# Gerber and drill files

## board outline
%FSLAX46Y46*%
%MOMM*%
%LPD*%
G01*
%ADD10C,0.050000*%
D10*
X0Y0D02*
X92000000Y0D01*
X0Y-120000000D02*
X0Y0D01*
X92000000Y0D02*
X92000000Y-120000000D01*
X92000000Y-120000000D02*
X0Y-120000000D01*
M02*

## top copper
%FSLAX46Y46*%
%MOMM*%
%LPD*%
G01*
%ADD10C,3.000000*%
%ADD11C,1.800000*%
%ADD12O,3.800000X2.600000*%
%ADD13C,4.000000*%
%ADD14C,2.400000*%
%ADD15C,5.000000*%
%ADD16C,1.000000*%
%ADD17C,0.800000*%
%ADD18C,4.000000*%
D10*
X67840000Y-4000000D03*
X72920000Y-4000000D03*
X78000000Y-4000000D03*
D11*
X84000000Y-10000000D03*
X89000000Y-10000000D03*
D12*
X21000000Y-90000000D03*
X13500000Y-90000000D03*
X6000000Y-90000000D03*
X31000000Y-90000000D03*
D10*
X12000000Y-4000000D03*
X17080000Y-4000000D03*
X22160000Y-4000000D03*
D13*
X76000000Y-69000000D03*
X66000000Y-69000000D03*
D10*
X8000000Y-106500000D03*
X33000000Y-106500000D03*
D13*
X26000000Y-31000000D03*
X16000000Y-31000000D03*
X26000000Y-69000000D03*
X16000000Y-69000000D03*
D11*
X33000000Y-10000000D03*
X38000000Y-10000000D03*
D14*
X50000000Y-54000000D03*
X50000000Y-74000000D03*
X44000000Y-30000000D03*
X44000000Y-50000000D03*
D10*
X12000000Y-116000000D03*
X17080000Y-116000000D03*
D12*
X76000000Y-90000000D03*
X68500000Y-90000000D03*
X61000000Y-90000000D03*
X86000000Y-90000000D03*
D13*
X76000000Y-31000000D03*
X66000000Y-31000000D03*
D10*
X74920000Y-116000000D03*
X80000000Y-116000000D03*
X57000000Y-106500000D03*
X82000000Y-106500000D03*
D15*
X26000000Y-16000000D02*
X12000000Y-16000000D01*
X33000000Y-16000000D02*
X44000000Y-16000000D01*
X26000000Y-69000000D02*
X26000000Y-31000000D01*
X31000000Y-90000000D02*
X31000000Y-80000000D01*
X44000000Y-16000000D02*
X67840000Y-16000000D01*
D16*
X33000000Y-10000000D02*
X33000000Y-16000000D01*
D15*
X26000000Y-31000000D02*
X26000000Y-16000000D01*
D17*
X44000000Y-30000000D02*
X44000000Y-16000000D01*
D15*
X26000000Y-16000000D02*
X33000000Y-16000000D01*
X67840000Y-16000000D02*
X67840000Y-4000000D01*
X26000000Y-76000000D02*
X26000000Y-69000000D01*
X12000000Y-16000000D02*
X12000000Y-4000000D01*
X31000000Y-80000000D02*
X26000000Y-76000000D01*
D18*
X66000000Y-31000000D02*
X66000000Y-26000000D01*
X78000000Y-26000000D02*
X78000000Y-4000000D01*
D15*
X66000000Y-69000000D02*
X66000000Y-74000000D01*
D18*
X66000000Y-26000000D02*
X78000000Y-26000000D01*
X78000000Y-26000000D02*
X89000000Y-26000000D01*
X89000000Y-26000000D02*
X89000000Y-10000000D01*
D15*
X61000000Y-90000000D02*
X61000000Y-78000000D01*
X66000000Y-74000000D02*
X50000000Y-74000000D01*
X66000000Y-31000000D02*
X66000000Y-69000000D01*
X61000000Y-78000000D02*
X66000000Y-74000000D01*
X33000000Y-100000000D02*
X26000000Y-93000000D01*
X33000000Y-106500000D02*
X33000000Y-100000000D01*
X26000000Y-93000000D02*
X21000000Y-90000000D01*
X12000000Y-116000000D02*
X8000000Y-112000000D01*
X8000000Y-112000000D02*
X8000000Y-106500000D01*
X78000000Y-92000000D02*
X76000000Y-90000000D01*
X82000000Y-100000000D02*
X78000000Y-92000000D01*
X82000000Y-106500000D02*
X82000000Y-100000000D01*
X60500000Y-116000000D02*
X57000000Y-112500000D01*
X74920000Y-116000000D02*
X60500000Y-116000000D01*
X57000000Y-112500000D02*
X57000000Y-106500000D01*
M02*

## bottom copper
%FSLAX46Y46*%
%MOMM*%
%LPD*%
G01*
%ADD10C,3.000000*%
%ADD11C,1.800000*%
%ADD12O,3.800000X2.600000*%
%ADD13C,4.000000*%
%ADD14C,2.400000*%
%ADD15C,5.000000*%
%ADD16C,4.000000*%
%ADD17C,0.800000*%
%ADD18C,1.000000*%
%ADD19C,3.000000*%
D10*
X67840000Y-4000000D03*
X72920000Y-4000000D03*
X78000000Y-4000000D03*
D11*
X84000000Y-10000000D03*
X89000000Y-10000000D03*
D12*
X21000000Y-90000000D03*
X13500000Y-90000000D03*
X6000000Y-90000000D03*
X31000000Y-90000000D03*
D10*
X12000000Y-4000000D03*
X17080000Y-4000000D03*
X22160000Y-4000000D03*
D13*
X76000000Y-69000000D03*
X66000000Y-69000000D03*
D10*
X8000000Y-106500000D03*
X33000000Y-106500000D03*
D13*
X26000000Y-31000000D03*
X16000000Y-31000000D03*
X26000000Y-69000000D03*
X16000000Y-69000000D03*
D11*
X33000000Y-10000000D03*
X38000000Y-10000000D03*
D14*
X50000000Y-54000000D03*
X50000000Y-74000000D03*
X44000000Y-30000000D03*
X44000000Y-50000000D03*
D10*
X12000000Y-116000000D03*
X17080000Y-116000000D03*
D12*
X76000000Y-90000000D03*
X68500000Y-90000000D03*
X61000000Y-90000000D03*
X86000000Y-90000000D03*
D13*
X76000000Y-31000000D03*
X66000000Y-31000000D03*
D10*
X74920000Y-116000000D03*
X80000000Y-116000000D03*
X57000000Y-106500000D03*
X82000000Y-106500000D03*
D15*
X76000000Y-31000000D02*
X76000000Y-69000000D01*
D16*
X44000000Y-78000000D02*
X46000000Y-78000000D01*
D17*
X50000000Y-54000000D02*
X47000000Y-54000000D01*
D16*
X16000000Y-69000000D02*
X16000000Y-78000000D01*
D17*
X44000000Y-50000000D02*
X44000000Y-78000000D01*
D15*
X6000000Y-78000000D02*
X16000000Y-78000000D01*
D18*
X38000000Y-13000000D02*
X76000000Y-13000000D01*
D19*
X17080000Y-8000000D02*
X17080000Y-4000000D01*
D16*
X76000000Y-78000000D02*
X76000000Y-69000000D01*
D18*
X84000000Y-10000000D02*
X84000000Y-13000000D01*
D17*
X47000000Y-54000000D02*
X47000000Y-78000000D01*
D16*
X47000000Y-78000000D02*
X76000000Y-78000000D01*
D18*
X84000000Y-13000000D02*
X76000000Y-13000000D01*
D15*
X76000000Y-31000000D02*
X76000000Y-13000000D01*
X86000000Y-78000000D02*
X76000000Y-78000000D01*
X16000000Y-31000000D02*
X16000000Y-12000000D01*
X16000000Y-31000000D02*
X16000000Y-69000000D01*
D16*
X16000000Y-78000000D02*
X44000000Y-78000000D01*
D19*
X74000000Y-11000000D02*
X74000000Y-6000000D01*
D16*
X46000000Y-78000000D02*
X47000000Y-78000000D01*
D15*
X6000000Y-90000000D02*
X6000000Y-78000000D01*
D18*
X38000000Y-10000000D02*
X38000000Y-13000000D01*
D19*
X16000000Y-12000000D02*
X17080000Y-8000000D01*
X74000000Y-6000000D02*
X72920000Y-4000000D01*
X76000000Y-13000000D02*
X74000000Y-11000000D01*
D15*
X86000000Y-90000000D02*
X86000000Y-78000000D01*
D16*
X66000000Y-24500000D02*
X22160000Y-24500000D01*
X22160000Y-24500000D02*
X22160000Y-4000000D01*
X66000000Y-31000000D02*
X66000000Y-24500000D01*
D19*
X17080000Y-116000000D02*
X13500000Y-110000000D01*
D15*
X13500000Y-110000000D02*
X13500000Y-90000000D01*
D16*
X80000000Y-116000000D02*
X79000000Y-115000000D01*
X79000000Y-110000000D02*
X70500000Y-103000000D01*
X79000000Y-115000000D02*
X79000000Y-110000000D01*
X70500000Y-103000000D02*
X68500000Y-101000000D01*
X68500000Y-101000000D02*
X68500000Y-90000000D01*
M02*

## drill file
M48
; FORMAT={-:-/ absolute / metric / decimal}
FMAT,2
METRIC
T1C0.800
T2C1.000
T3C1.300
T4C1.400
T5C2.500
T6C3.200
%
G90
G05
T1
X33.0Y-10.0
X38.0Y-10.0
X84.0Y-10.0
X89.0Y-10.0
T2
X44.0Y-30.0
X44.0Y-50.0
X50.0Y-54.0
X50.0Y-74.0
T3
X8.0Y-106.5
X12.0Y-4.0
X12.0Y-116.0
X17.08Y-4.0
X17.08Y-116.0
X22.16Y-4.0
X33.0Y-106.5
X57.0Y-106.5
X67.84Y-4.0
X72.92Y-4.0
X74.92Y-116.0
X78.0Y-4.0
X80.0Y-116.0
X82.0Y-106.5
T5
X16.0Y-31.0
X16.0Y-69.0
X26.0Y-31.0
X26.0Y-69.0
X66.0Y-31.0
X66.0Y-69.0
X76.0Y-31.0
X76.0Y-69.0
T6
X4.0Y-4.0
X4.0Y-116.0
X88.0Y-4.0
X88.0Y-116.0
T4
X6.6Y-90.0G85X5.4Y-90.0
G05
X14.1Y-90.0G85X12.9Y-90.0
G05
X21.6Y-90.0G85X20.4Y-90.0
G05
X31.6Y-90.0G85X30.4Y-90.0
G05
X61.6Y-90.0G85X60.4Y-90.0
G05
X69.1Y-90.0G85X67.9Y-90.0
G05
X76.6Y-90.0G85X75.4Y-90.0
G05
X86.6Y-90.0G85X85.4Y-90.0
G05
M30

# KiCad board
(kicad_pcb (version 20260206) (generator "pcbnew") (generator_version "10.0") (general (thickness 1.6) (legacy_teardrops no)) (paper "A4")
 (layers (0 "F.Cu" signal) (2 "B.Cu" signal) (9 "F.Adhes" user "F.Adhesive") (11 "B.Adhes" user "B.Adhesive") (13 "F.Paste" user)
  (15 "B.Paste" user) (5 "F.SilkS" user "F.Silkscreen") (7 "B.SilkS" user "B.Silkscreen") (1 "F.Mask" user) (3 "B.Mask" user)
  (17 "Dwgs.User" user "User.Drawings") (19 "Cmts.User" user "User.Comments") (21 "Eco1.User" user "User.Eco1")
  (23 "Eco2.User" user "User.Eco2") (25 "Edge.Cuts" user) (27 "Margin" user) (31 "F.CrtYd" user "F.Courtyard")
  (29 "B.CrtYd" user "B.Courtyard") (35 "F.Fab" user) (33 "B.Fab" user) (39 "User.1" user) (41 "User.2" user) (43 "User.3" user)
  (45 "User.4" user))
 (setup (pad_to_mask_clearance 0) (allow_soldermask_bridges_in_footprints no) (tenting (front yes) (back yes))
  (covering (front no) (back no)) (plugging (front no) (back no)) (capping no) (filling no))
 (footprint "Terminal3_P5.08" (layer "F.Cu") (at 67.84 4)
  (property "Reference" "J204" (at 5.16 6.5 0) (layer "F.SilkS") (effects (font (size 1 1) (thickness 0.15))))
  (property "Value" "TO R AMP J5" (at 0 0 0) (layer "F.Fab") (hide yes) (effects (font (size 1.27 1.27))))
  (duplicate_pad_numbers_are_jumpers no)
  (pad "1" thru_hole circle (at 0 0) (size 3 3) (drill 1.3) (layers "*.Cu" "*.Mask") (remove_unused_layers no) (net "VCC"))
  (pad "2" thru_hole circle (at 5.08 0) (size 3 3) (drill 1.3) (layers "*.Cu" "*.Mask") (remove_unused_layers no) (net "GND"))
  (pad "3" thru_hole circle (at 10.16 0) (size 3 3) (drill 1.3) (layers "*.Cu" "*.Mask") (remove_unused_layers no) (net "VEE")))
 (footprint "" (layer "F.Cu") (at 88 4)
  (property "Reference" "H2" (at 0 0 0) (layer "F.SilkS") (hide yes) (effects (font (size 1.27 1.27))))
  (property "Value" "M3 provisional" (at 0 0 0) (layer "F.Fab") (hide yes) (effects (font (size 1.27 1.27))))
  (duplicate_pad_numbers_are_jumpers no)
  (pad "" np_thru_hole circle (at 0 0) (size 3.2 3.2) (drill 3.2) (layers "*.Cu" "*.Mask")))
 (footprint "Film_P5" (layer "F.Cu") (at 84 10)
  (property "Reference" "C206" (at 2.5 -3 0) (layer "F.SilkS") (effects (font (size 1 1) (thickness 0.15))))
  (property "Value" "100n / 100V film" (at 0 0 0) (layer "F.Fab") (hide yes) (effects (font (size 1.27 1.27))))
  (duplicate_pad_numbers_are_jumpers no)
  (pad "1" thru_hole circle (at 0 0) (size 1.8 1.8) (drill 0.8) (layers "*.Cu" "*.Mask") (remove_unused_layers no) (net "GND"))
  (pad "2" thru_hole circle (at 5 0) (size 1.8 1.8) (drill 0.8) (layers "*.Cu" "*.Mask") (remove_unused_layers no) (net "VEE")))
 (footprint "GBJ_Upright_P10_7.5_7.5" (layer "F.Cu") (at 31 90 180)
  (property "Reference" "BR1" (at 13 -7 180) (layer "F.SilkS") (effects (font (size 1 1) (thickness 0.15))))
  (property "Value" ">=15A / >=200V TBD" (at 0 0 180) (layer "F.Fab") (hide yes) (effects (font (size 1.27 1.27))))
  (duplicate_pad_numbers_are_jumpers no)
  (pad "AC1" thru_hole oval (at 10 0 180) (size 3.8 2.6) (drill oval 2.6 1.4) (layers "*.Cu" "*.Mask") (remove_unused_layers no)
   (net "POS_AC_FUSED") (thermal_bridge_angle 45))
  (pad "AC2" thru_hole oval (at 17.5 0 180) (size 3.8 2.6) (drill oval 2.6 1.4) (layers "*.Cu" "*.Mask") (remove_unused_layers no)
   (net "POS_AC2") (thermal_bridge_angle 45))
  (pad "N" thru_hole oval (at 25 0 180) (size 3.8 2.6) (drill oval 2.6 1.4) (layers "*.Cu" "*.Mask") (remove_unused_layers no) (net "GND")
   (thermal_bridge_angle 45))
  (pad "P" thru_hole oval (at 0 0 180) (size 3.8 2.6) (drill oval 2.6 1.4) (layers "*.Cu" "*.Mask") (remove_unused_layers no) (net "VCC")
   (thermal_bridge_angle 45)))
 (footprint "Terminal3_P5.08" (layer "F.Cu") (at 12 4)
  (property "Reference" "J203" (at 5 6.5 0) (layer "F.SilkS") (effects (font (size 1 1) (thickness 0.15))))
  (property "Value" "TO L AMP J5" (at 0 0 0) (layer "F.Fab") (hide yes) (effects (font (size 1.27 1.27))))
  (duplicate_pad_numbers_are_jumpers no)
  (pad "1" thru_hole circle (at 0 0) (size 3 3) (drill 1.3) (layers "*.Cu" "*.Mask") (remove_unused_layers no) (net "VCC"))
  (pad "2" thru_hole circle (at 5.08 0) (size 3 3) (drill 1.3) (layers "*.Cu" "*.Mask") (remove_unused_layers no) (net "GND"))
  (pad "3" thru_hole circle (at 10.16 0) (size 3 3) (drill 1.3) (layers "*.Cu" "*.Mask") (remove_unused_layers no) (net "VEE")))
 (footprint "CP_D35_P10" (layer "F.Cu") (at 76 69 180)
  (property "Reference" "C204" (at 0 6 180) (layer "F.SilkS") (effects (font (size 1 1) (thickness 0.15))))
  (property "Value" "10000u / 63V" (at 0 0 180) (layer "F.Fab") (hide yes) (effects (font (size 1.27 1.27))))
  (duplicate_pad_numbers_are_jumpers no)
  (pad "1" thru_hole circle (at 0 0 180) (size 4 4) (drill 2.5) (layers "*.Cu" "*.Mask") (remove_unused_layers no) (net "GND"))
  (pad "2" thru_hole circle (at 10 0 180) (size 4 4) (drill 2.5) (layers "*.Cu" "*.Mask") (remove_unused_layers no) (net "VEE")))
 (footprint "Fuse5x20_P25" (layer "F.Cu") (at 8 106.5)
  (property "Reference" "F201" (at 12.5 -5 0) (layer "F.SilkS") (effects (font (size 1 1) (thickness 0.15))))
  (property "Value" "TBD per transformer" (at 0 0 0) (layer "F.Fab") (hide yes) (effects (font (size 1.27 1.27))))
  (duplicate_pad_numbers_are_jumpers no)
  (pad "1" thru_hole circle (at 0 0) (size 3 3) (drill 1.3) (layers "*.Cu" "*.Mask") (remove_unused_layers no) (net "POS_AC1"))
  (pad "2" thru_hole circle (at 25 0) (size 3 3) (drill 1.3) (layers "*.Cu" "*.Mask") (remove_unused_layers no) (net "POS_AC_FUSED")))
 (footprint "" (layer "F.Cu") (at 4 116)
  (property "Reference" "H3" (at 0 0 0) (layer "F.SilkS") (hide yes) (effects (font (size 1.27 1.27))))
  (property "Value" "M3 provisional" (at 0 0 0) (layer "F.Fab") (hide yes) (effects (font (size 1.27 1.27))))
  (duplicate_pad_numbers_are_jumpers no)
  (pad "" np_thru_hole circle (at 0 0) (size 3.2 3.2) (drill 3.2) (layers "*.Cu" "*.Mask")))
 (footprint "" (layer "F.Cu") (at 4 4)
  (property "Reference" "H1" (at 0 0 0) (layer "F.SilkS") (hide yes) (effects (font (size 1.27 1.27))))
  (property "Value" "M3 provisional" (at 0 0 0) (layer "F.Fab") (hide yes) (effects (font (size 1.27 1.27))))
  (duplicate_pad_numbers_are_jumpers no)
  (pad "" np_thru_hole circle (at 0 0) (size 3.2 3.2) (drill 3.2) (layers "*.Cu" "*.Mask")))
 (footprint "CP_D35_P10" (layer "F.Cu") (at 26 31 180)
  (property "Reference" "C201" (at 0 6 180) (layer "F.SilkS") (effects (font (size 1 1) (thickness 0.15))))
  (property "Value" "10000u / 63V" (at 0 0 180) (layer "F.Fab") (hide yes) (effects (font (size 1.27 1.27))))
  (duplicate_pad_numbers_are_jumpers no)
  (pad "1" thru_hole circle (at 0 0 180) (size 4 4) (drill 2.5) (layers "*.Cu" "*.Mask") (remove_unused_layers no) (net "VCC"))
  (pad "2" thru_hole circle (at 10 0 180) (size 4 4) (drill 2.5) (layers "*.Cu" "*.Mask") (remove_unused_layers no) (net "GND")))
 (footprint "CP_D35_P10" (layer "F.Cu") (at 26 69 180)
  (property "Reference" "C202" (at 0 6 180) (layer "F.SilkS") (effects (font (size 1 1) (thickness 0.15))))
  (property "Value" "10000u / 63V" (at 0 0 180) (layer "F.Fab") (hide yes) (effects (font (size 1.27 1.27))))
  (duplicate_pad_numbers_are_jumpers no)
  (pad "1" thru_hole circle (at 0 0 180) (size 4 4) (drill 2.5) (layers "*.Cu" "*.Mask") (remove_unused_layers no) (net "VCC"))
  (pad "2" thru_hole circle (at 10 0 180) (size 4 4) (drill 2.5) (layers "*.Cu" "*.Mask") (remove_unused_layers no) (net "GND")))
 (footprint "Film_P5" (layer "F.Cu") (at 33 10)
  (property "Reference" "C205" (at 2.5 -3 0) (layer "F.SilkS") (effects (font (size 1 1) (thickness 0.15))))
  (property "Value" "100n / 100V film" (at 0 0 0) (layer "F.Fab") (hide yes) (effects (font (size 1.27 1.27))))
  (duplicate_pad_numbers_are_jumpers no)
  (pad "1" thru_hole circle (at 0 0) (size 1.8 1.8) (drill 0.8) (layers "*.Cu" "*.Mask") (remove_unused_layers no) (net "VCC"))
  (pad "2" thru_hole circle (at 5 0) (size 1.8 1.8) (drill 0.8) (layers "*.Cu" "*.Mask") (remove_unused_layers no) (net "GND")))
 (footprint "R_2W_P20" (layer "F.Cu") (at 50 54 -90)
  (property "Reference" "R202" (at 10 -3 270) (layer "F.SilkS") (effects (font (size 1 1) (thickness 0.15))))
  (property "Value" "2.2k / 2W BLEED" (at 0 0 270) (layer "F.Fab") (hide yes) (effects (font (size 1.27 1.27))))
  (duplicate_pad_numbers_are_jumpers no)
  (pad "1" thru_hole circle (at 0 0 270) (size 2.4 2.4) (drill 1) (layers "*.Cu" "*.Mask") (remove_unused_layers no) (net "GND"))
  (pad "2" thru_hole circle (at 20 0 270) (size 2.4 2.4) (drill 1) (layers "*.Cu" "*.Mask") (remove_unused_layers no) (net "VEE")))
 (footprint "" (layer "F.Cu") (at 88 116)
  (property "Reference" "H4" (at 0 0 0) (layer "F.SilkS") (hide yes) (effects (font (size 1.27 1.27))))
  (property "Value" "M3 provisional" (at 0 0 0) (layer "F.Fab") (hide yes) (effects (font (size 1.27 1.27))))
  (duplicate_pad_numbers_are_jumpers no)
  (pad "" np_thru_hole circle (at 0 0) (size 3.2 3.2) (drill 3.2) (layers "*.Cu" "*.Mask")))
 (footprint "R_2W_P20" (layer "F.Cu") (at 44 30 -90)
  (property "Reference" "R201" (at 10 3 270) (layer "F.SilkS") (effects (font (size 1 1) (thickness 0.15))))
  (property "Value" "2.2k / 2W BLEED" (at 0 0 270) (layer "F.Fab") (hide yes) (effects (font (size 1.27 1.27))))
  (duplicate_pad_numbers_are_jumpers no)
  (pad "1" thru_hole circle (at 0 0 270) (size 2.4 2.4) (drill 1) (layers "*.Cu" "*.Mask") (remove_unused_layers no) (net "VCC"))
  (pad "2" thru_hole circle (at 20 0 270) (size 2.4 2.4) (drill 1) (layers "*.Cu" "*.Mask") (remove_unused_layers no) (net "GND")))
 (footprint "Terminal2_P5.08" (layer "F.Cu") (at 12 116)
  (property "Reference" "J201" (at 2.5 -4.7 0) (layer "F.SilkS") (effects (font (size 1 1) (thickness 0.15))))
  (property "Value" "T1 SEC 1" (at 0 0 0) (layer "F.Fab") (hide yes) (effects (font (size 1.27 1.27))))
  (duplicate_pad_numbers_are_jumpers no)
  (pad "1" thru_hole circle (at 0 0) (size 3 3) (drill 1.3) (layers "*.Cu" "*.Mask") (remove_unused_layers no) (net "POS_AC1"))
  (pad "2" thru_hole circle (at 5.08 0) (size 3 3) (drill 1.3) (layers "*.Cu" "*.Mask") (remove_unused_layers no) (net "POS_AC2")))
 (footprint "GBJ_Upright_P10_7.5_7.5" (layer "F.Cu") (at 86 90 180)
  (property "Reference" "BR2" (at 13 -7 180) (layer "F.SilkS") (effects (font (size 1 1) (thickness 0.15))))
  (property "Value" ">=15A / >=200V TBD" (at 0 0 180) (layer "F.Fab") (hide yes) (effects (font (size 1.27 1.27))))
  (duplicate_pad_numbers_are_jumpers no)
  (pad "AC1" thru_hole oval (at 10 0 180) (size 3.8 2.6) (drill oval 2.6 1.4) (layers "*.Cu" "*.Mask") (remove_unused_layers no)
   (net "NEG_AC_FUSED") (thermal_bridge_angle 45))
  (pad "AC2" thru_hole oval (at 17.5 0 180) (size 3.8 2.6) (drill oval 2.6 1.4) (layers "*.Cu" "*.Mask") (remove_unused_layers no)
   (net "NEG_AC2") (thermal_bridge_angle 45))
  (pad "N" thru_hole oval (at 25 0 180) (size 3.8 2.6) (drill oval 2.6 1.4) (layers "*.Cu" "*.Mask") (remove_unused_layers no) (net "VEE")
   (thermal_bridge_angle 45))
  (pad "P" thru_hole oval (at 0 0 180) (size 3.8 2.6) (drill oval 2.6 1.4) (layers "*.Cu" "*.Mask") (remove_unused_layers no) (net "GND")
   (thermal_bridge_angle 45)))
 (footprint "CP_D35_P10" (layer "F.Cu") (at 76 31 180)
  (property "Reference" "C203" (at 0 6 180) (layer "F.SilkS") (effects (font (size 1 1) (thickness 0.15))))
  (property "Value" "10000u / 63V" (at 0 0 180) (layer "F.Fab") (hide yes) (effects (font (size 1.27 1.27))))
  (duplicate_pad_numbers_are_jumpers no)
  (pad "1" thru_hole circle (at 0 0 180) (size 4 4) (drill 2.5) (layers "*.Cu" "*.Mask") (remove_unused_layers no) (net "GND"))
  (pad "2" thru_hole circle (at 10 0 180) (size 4 4) (drill 2.5) (layers "*.Cu" "*.Mask") (remove_unused_layers no) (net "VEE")))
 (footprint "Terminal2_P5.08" (layer "F.Cu") (at 74.92 116)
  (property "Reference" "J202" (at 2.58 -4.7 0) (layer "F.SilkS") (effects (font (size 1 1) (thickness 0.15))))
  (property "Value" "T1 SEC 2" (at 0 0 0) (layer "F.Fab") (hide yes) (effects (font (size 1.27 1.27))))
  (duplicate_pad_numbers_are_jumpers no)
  (pad "1" thru_hole circle (at 0 0) (size 3 3) (drill 1.3) (layers "*.Cu" "*.Mask") (remove_unused_layers no) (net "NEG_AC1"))
  (pad "2" thru_hole circle (at 5.08 0) (size 3 3) (drill 1.3) (layers "*.Cu" "*.Mask") (remove_unused_layers no) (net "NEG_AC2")))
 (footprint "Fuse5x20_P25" (layer "F.Cu") (at 57 106.5)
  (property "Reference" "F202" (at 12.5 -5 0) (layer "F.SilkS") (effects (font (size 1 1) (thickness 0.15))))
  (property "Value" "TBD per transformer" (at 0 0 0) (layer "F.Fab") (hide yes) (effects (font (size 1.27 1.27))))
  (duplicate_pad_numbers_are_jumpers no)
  (pad "1" thru_hole circle (at 0 0) (size 3 3) (drill 1.3) (layers "*.Cu" "*.Mask") (remove_unused_layers no) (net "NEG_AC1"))
  (pad "2" thru_hole circle (at 25 0) (size 3 3) (drill 1.3) (layers "*.Cu" "*.Mask") (remove_unused_layers no) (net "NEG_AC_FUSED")))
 (gr_line (start 0 0) (end 92 0) (stroke (width 0.05) (type default)) (layer "Edge.Cuts"))
 (gr_line (start 0 120) (end 0 0) (stroke (width 0.05) (type default)) (layer "Edge.Cuts"))
 (gr_line (start 92 0) (end 92 120) (stroke (width 0.05) (type default)) (layer "Edge.Cuts"))
 (gr_line (start 92 120) (end 0 120) (stroke (width 0.05) (type default)) (layer "Edge.Cuts"))
 (segment (start 26 16) (end 12 16) (width 5) (layer "F.Cu") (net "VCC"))
 (segment (start 33 16) (end 44 16) (width 5) (layer "F.Cu") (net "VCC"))
 (segment (start 26 69) (end 26 31) (width 5) (layer "F.Cu") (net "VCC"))
 (segment (start 31 90) (end 31 80) (width 5) (layer "F.Cu") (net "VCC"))
 (segment (start 44 16) (end 67.84 16) (width 5) (layer "F.Cu") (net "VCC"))
 (segment (start 33 10) (end 33 16) (width 1) (layer "F.Cu") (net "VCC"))
 (segment (start 26 31) (end 26 16) (width 5) (layer "F.Cu") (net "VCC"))
 (segment (start 44 30) (end 44 16) (width 0.8) (layer "F.Cu") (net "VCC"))
 (segment (start 26 16) (end 33 16) (width 5) (layer "F.Cu") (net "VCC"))
 (segment (start 67.84 16) (end 67.84 4) (width 5) (layer "F.Cu") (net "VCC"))
 (segment (start 26 76) (end 26 69) (width 5) (layer "F.Cu") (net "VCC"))
 (segment (start 12 16) (end 12 4) (width 5) (layer "F.Cu") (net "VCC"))
 (segment (start 31 80) (end 26 76) (width 5) (layer "F.Cu") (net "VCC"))
 (segment (start 76 31) (end 76 69) (width 5) (layer "B.Cu") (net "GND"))
 (segment (start 44 78) (end 46 78) (width 4) (layer "B.Cu") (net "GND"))
 (segment (start 50 54) (end 47 54) (width 0.8) (layer "B.Cu") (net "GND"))
 (segment (start 16 69) (end 16 78) (width 4) (layer "B.Cu") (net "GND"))
 (segment (start 44 50) (end 44 78) (width 0.8) (layer "B.Cu") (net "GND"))
 (segment (start 6 78) (end 16 78) (width 5) (layer "B.Cu") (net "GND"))
 (segment (start 38 13) (end 76 13) (width 1) (layer "B.Cu") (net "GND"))
 (segment (start 17.08 8) (end 17.08 4) (width 3) (layer "B.Cu") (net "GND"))
 (segment (start 76 78) (end 76 69) (width 4) (layer "B.Cu") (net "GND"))
 (segment (start 84 10) (end 84 13) (width 1) (layer "B.Cu") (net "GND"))
 (segment (start 47 54) (end 47 78) (width 0.8) (layer "B.Cu") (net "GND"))
 (segment (start 47 78) (end 76 78) (width 4) (layer "B.Cu") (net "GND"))
 (segment (start 84 13) (end 76 13) (width 1) (layer "B.Cu") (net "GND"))
 (segment (start 76 31) (end 76 13) (width 5) (layer "B.Cu") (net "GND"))
 (segment (start 86 78) (end 76 78) (width 5) (layer "B.Cu") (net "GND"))
 (segment (start 16 31) (end 16 12) (width 5) (layer "B.Cu") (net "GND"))
 (segment (start 16 31) (end 16 69) (width 5) (layer "B.Cu") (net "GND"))
 (segment (start 16 78) (end 44 78) (width 4) (layer "B.Cu") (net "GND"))
 (segment (start 74 11) (end 74 6) (width 3) (layer "B.Cu") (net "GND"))
 (segment (start 46 78) (end 47 78) (width 4) (layer "B.Cu") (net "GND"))
 (segment (start 6 90) (end 6 78) (width 5) (layer "B.Cu") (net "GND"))
 (segment (start 38 10) (end 38 13) (width 1) (layer "B.Cu") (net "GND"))
 (segment (start 16 12) (end 17.08 8) (width 3) (layer "B.Cu") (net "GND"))
 (segment (start 74 6) (end 72.92 4) (width 3) (layer "B.Cu") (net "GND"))
 (segment (start 76 13) (end 74 11) (width 3) (layer "B.Cu") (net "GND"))
 (segment (start 86 90) (end 86 78) (width 5) (layer "B.Cu") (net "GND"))
 (segment (start 66 31) (end 66 26) (width 4) (layer "F.Cu") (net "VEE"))
 (segment (start 78 26) (end 78 4) (width 4) (layer "F.Cu") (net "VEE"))
 (segment (start 66 69) (end 66 74) (width 5) (layer "F.Cu") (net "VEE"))
 (segment (start 66 26) (end 78 26) (width 4) (layer "F.Cu") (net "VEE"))
 (segment (start 78 26) (end 89 26) (width 4) (layer "F.Cu") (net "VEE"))
 (segment (start 89 26) (end 89 10) (width 4) (layer "F.Cu") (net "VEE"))
 (segment (start 61 90) (end 61 78) (width 5) (layer "F.Cu") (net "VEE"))
 (segment (start 66 74) (end 50 74) (width 5) (layer "F.Cu") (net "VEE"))
 (segment (start 66 31) (end 66 69) (width 5) (layer "F.Cu") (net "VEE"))
 (segment (start 61 78) (end 66 74) (width 5) (layer "F.Cu") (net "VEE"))
 (segment (start 66 24.5) (end 22.16 24.5) (width 4) (layer "B.Cu") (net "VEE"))
 (segment (start 22.16 24.5) (end 22.16 4) (width 4) (layer "B.Cu") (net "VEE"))
 (segment (start 66 31) (end 66 24.5) (width 4) (layer "B.Cu") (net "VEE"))
 (segment (start 33 100) (end 26 93) (width 5) (layer "F.Cu") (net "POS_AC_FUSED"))
 (segment (start 33 106.5) (end 33 100) (width 5) (layer "F.Cu") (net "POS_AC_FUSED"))
 (segment (start 26 93) (end 21 90) (width 5) (layer "F.Cu") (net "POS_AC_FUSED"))
 (segment (start 17.08 116) (end 13.5 110) (width 3) (layer "B.Cu") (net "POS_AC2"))
 (segment (start 13.5 110) (end 13.5 90) (width 5) (layer "B.Cu") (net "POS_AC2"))
 (segment (start 12 116) (end 8 112) (width 5) (layer "F.Cu") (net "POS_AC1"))
 (segment (start 8 112) (end 8 106.5) (width 5) (layer "F.Cu") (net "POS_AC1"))
 (segment (start 78 92) (end 76 90) (width 5) (layer "F.Cu") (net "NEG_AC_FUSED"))
 (segment (start 82 100) (end 78 92) (width 5) (layer "F.Cu") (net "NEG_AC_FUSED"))
 (segment (start 82 106.5) (end 82 100) (width 5) (layer "F.Cu") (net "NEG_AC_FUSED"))
 (segment (start 80 116) (end 79 115) (width 4) (layer "B.Cu") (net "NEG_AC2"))
 (segment (start 79 110) (end 70.5 103) (width 4) (layer "B.Cu") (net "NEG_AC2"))
 (segment (start 79 115) (end 79 110) (width 4) (layer "B.Cu") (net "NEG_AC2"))
 (segment (start 70.5 103) (end 68.5 101) (width 4) (layer "B.Cu") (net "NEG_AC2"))
 (segment (start 68.5 101) (end 68.5 90) (width 4) (layer "B.Cu") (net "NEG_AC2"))
 (segment (start 60.5 116) (end 57 112.5) (width 5) (layer "F.Cu") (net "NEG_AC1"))
 (segment (start 74.92 116) (end 60.5 116) (width 5) (layer "F.Cu") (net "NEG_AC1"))
 (segment (start 57 112.5) (end 57 106.5) (width 5) (layer "F.Cu") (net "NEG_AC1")))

